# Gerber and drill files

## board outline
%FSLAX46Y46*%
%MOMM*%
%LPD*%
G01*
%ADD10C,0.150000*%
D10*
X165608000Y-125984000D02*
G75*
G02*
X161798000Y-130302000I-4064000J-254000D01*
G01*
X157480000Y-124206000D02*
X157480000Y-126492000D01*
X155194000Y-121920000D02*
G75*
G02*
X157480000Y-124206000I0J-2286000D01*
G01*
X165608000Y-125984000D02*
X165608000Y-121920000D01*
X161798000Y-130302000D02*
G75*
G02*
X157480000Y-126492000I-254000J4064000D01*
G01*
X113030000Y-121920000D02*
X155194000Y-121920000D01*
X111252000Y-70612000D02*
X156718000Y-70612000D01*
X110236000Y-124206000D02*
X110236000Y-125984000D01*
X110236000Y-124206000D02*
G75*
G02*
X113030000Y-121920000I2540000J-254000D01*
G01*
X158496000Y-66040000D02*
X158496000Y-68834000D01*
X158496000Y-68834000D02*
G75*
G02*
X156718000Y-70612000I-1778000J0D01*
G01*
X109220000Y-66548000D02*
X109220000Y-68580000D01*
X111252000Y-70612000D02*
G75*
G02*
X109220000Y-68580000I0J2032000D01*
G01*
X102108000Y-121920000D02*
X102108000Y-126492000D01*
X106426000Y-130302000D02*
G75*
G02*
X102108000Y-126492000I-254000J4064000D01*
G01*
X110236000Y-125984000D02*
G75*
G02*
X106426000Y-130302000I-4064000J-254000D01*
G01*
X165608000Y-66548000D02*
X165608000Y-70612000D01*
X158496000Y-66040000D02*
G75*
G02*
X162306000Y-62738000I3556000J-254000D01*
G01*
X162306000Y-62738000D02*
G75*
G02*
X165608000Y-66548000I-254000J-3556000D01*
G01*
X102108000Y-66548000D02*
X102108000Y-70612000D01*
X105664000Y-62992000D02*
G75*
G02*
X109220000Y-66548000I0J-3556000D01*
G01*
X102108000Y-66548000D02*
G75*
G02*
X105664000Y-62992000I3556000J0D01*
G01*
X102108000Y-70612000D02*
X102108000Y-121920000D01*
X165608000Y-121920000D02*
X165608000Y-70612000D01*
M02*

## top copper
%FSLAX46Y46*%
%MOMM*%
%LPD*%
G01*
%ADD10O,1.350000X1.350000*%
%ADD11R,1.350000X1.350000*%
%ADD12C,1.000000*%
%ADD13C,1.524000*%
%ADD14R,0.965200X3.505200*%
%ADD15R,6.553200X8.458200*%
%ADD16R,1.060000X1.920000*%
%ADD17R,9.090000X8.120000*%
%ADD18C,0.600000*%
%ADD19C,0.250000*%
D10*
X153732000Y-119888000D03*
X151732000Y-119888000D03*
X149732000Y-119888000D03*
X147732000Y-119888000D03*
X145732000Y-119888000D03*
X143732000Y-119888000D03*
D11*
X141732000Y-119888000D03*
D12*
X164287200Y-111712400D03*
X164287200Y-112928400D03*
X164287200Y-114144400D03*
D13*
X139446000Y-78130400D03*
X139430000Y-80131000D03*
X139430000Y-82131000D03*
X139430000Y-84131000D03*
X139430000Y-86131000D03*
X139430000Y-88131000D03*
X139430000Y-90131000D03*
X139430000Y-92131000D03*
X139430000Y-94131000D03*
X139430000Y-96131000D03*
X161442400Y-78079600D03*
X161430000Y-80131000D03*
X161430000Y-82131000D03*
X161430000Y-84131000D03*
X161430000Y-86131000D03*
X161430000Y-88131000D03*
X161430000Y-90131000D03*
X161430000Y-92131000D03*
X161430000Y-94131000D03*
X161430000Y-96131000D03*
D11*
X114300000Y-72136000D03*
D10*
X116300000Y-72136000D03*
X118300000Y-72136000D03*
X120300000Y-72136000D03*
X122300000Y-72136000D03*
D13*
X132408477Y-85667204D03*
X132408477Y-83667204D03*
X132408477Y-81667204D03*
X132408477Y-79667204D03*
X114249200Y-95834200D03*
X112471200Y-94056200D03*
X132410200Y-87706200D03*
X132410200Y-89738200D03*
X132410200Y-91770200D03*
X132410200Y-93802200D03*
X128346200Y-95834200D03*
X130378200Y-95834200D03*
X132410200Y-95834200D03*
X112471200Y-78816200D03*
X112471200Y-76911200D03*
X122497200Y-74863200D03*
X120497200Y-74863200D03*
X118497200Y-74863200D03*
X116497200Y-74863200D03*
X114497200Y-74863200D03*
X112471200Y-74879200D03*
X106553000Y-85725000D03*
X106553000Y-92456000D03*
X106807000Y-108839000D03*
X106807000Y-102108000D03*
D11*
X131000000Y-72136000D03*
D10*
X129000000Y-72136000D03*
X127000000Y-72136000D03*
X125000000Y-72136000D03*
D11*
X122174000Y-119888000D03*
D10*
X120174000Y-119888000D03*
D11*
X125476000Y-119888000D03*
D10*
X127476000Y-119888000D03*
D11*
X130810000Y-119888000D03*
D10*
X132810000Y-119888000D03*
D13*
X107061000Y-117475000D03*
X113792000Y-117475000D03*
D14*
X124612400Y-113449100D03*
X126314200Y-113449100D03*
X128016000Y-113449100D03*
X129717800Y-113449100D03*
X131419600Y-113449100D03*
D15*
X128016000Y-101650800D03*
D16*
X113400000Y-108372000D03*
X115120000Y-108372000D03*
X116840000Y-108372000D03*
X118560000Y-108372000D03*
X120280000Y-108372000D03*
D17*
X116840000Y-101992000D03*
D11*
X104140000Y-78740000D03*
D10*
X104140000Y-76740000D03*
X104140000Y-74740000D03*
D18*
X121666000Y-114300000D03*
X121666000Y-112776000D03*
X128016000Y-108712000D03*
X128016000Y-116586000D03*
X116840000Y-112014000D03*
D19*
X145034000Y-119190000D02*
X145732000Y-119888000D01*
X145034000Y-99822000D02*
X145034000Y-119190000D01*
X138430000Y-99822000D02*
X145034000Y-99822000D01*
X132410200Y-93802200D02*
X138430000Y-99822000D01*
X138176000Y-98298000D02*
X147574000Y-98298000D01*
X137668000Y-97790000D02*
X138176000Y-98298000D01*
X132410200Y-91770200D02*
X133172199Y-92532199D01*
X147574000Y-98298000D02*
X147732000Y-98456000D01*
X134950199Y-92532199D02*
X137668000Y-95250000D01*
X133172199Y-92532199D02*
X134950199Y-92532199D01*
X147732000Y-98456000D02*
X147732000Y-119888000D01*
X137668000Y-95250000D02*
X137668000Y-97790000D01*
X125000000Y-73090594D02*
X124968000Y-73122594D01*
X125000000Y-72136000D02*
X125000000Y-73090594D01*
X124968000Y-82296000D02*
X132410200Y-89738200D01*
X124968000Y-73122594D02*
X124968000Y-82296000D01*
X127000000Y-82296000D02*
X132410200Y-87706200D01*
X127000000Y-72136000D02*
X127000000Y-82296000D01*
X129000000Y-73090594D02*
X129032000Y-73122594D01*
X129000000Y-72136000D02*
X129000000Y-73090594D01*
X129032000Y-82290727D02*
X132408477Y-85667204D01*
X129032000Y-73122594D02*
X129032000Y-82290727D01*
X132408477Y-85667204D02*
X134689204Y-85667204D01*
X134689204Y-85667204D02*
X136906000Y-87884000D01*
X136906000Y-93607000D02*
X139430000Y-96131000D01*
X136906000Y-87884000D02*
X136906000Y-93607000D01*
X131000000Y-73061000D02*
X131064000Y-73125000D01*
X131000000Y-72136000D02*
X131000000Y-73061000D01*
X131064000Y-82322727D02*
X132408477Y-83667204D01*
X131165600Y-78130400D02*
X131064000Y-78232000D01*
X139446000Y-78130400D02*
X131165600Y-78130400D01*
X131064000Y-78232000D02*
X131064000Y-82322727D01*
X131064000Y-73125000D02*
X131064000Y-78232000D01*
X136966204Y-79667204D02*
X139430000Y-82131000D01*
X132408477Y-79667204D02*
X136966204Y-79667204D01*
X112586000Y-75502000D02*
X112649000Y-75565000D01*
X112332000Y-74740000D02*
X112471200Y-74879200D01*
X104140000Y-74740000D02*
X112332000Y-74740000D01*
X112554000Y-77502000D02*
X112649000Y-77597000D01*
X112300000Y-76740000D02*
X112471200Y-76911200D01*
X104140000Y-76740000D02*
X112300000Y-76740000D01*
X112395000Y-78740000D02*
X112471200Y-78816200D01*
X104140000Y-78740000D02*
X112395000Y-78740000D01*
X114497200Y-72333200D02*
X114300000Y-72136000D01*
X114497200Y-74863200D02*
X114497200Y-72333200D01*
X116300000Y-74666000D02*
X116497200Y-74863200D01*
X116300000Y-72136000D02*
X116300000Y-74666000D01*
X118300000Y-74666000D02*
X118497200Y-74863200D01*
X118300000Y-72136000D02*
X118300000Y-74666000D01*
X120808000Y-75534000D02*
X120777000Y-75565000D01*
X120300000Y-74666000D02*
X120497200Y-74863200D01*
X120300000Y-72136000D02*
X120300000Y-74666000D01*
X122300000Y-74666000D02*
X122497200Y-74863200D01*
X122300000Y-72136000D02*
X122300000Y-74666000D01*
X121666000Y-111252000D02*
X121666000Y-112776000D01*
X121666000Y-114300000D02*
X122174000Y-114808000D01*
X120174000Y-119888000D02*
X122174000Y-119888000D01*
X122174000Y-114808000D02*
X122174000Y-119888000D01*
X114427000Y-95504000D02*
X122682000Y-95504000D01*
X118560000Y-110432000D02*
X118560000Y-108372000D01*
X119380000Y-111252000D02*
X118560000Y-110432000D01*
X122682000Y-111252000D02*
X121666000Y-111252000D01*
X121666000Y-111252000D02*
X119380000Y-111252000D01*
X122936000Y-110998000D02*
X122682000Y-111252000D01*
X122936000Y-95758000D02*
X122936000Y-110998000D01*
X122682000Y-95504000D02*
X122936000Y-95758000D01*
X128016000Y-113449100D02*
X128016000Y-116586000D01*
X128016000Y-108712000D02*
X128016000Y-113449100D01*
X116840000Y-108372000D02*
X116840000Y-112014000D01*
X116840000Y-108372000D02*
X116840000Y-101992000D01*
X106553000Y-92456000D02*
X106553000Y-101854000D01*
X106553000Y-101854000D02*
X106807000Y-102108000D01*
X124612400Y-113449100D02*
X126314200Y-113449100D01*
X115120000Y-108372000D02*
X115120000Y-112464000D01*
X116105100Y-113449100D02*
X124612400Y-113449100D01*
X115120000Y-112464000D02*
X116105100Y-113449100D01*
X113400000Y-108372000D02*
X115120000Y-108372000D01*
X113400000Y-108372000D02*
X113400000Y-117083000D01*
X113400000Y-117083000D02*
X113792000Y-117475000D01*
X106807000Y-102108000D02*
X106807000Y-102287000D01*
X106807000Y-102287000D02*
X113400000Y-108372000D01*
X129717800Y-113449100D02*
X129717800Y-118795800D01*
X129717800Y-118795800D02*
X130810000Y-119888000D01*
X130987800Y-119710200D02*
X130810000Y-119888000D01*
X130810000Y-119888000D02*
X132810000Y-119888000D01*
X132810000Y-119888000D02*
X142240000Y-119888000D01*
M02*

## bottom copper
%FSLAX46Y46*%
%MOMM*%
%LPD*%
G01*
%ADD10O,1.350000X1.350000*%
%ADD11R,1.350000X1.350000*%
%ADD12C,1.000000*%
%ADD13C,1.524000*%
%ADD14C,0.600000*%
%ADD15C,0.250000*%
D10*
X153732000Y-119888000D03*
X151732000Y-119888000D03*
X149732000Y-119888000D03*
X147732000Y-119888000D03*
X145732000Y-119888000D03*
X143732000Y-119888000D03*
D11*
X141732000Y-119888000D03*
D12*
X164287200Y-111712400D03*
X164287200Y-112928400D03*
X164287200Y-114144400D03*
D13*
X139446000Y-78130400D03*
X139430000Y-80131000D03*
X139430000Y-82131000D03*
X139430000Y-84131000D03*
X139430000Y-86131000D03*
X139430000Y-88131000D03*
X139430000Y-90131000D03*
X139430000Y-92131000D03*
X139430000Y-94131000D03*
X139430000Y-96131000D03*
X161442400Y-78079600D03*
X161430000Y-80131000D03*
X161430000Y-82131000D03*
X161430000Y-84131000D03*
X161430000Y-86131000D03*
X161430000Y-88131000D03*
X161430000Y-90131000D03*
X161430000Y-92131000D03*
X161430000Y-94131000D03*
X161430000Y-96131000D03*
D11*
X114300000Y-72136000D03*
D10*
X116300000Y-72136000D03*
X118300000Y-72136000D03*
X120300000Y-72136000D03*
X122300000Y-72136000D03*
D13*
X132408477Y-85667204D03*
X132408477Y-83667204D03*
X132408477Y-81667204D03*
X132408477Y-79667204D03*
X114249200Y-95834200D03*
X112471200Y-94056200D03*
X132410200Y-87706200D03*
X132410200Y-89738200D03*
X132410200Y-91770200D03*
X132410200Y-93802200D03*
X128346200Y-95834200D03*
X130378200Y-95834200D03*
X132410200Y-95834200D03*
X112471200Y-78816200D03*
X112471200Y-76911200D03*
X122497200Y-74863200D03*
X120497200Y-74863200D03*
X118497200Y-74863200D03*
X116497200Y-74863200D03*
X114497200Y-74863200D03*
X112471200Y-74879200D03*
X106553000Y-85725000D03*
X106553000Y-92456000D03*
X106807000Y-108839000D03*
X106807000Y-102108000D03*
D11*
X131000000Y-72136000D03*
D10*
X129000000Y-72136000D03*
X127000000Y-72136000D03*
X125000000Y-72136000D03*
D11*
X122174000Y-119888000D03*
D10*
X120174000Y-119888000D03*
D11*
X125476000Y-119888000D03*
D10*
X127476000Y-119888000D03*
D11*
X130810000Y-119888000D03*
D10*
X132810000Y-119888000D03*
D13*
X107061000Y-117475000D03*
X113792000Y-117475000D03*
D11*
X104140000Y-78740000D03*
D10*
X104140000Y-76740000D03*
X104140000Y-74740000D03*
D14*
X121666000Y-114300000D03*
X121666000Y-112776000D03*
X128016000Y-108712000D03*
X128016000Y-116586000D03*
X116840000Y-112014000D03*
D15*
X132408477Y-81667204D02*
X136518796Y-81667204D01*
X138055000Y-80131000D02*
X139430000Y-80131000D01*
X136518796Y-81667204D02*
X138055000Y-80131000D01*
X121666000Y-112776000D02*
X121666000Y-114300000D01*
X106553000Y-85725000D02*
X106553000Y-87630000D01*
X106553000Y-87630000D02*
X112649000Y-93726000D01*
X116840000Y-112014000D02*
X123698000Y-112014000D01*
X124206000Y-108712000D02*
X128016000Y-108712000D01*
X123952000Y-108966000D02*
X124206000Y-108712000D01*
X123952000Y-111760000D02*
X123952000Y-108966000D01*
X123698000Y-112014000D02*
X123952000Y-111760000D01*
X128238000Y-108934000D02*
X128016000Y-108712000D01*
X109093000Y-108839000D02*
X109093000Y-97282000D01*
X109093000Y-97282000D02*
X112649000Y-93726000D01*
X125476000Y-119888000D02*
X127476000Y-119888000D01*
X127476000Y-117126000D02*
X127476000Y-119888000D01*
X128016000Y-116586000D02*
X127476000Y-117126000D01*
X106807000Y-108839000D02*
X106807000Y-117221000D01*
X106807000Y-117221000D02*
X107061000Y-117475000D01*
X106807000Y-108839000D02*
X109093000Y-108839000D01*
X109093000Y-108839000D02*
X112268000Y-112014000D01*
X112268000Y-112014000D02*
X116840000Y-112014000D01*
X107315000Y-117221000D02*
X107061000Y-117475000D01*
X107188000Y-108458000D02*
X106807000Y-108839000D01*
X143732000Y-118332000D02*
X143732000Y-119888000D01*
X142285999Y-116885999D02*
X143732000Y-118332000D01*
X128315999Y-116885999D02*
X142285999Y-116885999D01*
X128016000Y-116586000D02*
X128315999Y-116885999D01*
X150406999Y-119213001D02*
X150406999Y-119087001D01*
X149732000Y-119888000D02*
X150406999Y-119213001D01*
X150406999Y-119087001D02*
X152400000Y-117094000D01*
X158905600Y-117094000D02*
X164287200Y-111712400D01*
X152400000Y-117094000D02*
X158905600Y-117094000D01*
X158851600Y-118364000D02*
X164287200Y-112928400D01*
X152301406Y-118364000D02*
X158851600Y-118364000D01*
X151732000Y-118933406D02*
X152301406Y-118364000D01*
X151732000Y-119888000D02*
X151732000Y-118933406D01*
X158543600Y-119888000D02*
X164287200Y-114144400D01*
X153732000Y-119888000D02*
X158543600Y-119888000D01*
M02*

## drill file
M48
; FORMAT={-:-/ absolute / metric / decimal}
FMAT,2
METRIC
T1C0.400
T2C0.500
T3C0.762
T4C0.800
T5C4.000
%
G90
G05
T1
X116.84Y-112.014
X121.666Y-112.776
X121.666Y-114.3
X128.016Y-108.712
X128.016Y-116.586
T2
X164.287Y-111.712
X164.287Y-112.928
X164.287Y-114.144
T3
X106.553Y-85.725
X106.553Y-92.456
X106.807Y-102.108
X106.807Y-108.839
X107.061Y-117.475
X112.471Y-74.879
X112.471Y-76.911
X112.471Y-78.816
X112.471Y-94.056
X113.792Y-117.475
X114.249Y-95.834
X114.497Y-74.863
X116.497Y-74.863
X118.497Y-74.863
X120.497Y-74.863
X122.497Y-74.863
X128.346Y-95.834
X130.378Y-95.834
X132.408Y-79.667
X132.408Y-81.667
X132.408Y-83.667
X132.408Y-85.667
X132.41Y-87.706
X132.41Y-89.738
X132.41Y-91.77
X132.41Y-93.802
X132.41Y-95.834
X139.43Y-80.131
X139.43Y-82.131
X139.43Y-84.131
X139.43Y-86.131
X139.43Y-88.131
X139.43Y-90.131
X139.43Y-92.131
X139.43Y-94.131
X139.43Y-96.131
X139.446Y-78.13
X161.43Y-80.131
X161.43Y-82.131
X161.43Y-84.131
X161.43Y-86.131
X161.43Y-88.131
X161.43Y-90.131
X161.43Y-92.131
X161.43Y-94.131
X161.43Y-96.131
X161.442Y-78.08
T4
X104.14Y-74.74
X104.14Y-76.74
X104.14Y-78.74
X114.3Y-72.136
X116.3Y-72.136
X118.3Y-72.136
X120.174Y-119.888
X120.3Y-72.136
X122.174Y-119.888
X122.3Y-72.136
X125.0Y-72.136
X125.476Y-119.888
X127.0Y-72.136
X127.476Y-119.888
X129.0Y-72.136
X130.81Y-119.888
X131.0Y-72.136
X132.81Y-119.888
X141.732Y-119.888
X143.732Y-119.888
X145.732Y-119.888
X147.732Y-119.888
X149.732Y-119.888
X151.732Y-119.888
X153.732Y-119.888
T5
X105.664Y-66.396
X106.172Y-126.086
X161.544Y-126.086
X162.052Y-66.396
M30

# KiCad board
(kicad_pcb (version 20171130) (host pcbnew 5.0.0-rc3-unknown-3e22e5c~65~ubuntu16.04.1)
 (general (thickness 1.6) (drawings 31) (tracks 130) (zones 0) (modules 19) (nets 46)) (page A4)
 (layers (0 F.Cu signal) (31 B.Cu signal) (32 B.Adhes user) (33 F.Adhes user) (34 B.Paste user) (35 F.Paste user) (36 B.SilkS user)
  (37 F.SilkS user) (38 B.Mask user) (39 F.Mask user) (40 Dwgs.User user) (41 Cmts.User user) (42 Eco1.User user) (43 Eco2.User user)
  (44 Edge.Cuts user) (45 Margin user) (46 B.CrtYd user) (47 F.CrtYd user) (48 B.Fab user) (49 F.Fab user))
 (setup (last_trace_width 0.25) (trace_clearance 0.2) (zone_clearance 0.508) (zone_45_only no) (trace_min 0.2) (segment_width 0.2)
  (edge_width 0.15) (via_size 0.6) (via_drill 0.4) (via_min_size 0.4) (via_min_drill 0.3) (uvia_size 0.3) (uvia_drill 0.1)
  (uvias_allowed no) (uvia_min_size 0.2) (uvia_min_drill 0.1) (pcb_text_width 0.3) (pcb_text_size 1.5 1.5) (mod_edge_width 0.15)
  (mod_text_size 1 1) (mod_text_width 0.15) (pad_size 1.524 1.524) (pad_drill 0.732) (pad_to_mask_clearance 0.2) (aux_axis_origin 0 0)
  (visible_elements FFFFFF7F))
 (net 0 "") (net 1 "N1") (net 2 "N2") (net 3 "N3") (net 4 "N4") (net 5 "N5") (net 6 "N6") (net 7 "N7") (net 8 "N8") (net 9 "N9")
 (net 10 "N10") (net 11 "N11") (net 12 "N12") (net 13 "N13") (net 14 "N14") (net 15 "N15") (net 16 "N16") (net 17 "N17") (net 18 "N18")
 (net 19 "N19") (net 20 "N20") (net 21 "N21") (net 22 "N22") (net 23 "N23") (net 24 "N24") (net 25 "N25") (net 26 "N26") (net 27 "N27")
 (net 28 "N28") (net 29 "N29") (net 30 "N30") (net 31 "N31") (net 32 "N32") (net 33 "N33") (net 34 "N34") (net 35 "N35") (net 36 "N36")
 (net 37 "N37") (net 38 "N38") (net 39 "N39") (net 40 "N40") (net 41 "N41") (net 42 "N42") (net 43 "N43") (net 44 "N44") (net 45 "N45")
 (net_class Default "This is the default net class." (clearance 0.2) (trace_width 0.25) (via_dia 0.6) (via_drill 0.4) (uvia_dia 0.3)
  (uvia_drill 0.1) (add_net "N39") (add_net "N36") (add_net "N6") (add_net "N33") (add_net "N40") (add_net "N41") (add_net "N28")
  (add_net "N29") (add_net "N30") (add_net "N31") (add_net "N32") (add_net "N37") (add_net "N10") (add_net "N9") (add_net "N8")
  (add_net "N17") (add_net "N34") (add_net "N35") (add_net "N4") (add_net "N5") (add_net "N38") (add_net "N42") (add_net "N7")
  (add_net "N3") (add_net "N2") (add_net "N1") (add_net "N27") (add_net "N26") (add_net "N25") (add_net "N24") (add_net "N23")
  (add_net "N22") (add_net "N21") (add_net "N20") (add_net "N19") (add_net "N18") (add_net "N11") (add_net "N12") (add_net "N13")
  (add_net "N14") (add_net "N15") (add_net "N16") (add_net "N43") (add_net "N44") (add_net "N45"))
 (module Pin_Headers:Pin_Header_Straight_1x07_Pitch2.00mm (layer F.Cu) (at 141.732 119.888 90)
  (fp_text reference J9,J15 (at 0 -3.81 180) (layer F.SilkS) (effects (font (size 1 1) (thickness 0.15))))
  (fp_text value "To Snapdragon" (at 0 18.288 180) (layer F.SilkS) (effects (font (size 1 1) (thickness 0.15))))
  (pad 5 thru_hole oval (at 0 12 90) (size 1.35 1.35) (drill 0.8) (layers *.Cu *.Mask) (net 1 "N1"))
  (pad 4 thru_hole oval (at 0 10 90) (size 1.35 1.35) (drill 0.8) (layers *.Cu *.Mask) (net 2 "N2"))
  (pad 3 thru_hole oval (at 0 8 90) (size 1.35 1.35) (drill 0.8) (layers *.Cu *.Mask) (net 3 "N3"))
  (pad 6 thru_hole oval (at 0 6 90) (size 1.35 1.35) (drill 0.8) (layers *.Cu *.Mask) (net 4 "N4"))
  (pad 7 thru_hole oval (at 0 4 90) (size 1.35 1.35) (drill 0.8) (layers *.Cu *.Mask) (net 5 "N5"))
  (pad 2 thru_hole oval (at 0 2 90) (size 1.35 1.35) (drill 0.8) (layers *.Cu *.Mask) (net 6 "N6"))
  (pad 1 thru_hole rect (at 0 0 90) (size 1.35 1.35) (drill 0.8) (layers *.Cu *.Mask) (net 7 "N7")))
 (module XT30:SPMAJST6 (layer F.Cu) (at 163.576 113.792 270)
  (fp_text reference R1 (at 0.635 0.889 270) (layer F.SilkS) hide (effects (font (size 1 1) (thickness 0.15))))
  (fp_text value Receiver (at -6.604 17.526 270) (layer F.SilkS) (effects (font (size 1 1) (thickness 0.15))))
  (pad 1 thru_hole circle (at -2.0796 -0.7112 270) (size 1 1) (drill 0.5) (layers *.Cu *.Mask) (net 3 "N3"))
  (pad 2 thru_hole circle (at -0.8636 -0.7112 270) (size 1 1) (drill 0.5) (layers *.Cu *.Mask) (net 2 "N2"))
  (pad 3 thru_hole circle (at 0.3524 -0.7112 270) (size 1 1) (drill 0.5) (layers *.Cu *.Mask) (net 1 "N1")))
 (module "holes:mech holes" (layer F.Cu) (at 162.052 129.286)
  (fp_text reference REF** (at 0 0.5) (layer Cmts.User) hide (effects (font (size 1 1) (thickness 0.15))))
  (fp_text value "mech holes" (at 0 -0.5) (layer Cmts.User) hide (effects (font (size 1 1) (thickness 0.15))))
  (pad "" np_thru_hole circle (at -0.508 -3.2004) (size 4 4) (drill 4) (layers *.Cu *.Mask)))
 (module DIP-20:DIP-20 (layer F.Cu) (at 138.176 104.14)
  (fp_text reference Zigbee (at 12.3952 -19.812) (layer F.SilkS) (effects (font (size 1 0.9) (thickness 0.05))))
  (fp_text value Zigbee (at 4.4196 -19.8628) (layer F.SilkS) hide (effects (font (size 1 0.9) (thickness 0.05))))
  (pad 1 thru_hole circle (at 1.27 -26.0096) (size 1.524 1.524) (drill 0.762) (layers *.Cu *.Mask F.SilkS) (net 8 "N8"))
  (pad 2 thru_hole circle (at 1.254 -24.009) (size 1.524 1.524) (drill 0.762) (layers *.Cu *.Mask F.SilkS) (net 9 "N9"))
  (pad 3 thru_hole circle (at 1.254 -22.009) (size 1.524 1.524) (drill 0.762) (layers *.Cu *.Mask F.SilkS) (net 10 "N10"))
  (pad 4 thru_hole circle (at 1.254 -20.009) (size 1.524 1.524) (drill 0.762) (layers *.Cu *.Mask F.SilkS) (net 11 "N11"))
  (pad 5 thru_hole circle (at 1.254 -18.009) (size 1.524 1.524) (drill 0.762) (layers *.Cu *.Mask F.SilkS) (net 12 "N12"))
  (pad 6 thru_hole circle (at 1.254 -16.009) (size 1.524 1.524) (drill 0.762) (layers *.Cu *.Mask F.SilkS) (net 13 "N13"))
  (pad 7 thru_hole circle (at 1.254 -14.009) (size 1.524 1.524) (drill 0.762) (layers *.Cu *.Mask F.SilkS) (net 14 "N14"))
  (pad 8 thru_hole circle (at 1.254 -12.009) (size 1.524 1.524) (drill 0.762) (layers *.Cu *.Mask F.SilkS) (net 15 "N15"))
  (pad 9 thru_hole circle (at 1.254 -10.009) (size 1.524 1.524) (drill 0.762) (layers *.Cu *.Mask F.SilkS) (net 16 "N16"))
  (pad 10 thru_hole circle (at 1.254 -8.009) (size 1.524 1.524) (drill 0.762) (layers *.Cu *.Mask F.SilkS) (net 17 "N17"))
  (pad 20 thru_hole circle (at 23.2664 -26.0604) (size 1.524 1.524) (drill 0.762) (layers *.Cu *.Mask F.SilkS) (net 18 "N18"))
  (pad 19 thru_hole circle (at 23.254 -24.009) (size 1.524 1.524) (drill 0.762) (layers *.Cu *.Mask F.SilkS) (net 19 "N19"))
  (pad 18 thru_hole circle (at 23.254 -22.009) (size 1.524 1.524) (drill 0.762) (layers *.Cu *.Mask F.SilkS) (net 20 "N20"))
  (pad 17 thru_hole circle (at 23.254 -20.009) (size 1.524 1.524) (drill 0.762) (layers *.Cu *.Mask F.SilkS) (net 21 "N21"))
  (pad 16 thru_hole circle (at 23.254 -18.009) (size 1.524 1.524) (drill 0.762) (layers *.Cu *.Mask F.SilkS) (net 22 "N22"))
  (pad 15 thru_hole circle (at 23.254 -16.009) (size 1.524 1.524) (drill 0.762) (layers *.Cu *.Mask F.SilkS) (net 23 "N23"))
  (pad 14 thru_hole circle (at 23.254 -14.009) (size 1.524 1.524) (drill 0.762) (layers *.Cu *.Mask F.SilkS) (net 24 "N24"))
  (pad 13 thru_hole circle (at 23.254 -12.009) (size 1.524 1.524) (drill 0.762) (layers *.Cu *.Mask F.SilkS) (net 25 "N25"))
  (pad 12 thru_hole circle (at 23.254 -10.009) (size 1.524 1.524) (drill 0.762) (layers *.Cu *.Mask F.SilkS) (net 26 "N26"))
  (pad 11 thru_hole circle (at 23.254 -8.009) (size 1.524 1.524) (drill 0.762) (layers *.Cu *.Mask F.SilkS) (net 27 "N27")))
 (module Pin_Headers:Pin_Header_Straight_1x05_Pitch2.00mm (layer F.Cu) (at 114.3 72.136 90)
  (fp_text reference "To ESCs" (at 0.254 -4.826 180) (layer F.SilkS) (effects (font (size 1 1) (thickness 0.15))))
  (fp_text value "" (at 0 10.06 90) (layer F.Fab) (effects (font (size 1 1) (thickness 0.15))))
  (pad 1 thru_hole rect (at 0 0 90) (size 1.35 1.35) (drill 0.8) (layers *.Cu *.Mask) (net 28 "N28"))
  (pad 2 thru_hole oval (at 0 2 90) (size 1.35 1.35) (drill 0.8) (layers *.Cu *.Mask) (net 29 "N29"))
  (pad 3 thru_hole oval (at 0 4 90) (size 1.35 1.35) (drill 0.8) (layers *.Cu *.Mask) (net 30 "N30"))
  (pad 4 thru_hole oval (at 0 6 90) (size 1.35 1.35) (drill 0.8) (layers *.Cu *.Mask) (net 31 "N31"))
  (pad 5 thru_hole oval (at 0 8 90) (size 1.35 1.35) (drill 0.8) (layers *.Cu *.Mask) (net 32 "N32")))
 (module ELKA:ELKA (layer F.Cu) (at 121.666 85.852)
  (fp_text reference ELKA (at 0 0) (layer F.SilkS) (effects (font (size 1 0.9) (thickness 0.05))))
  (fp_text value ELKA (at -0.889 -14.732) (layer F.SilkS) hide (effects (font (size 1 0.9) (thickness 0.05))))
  (pad D thru_hole circle (at 10.742477 -0.184796) (size 1.524 1.524) (drill 0.762) (layers *.Cu *.Mask B.SilkS) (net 17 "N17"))
  (pad C thru_hole circle (at 10.742477 -2.184796) (size 1.524 1.524) (drill 0.762) (layers *.Cu *.Mask B.SilkS) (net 8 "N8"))
  (pad B thru_hole circle (at 10.742477 -4.184796) (size 1.524 1.524) (drill 0.762) (layers *.Cu *.Mask B.SilkS) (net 9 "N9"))
  (pad A thru_hole circle (at 10.742477 -6.184796) (size 1.524 1.524) (drill 0.762) (layers *.Cu *.Mask B.SilkS) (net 10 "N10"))
  (pad 12 thru_hole circle (at -7.4168 9.9822) (size 1.524 1.524) (drill 0.762) (layers *.Cu *.Mask B.SilkS) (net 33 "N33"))
  (pad 11 thru_hole circle (at -9.1948 8.2042 270) (size 1.524 1.524) (drill 0.762) (layers *.Cu *.Mask B.SilkS) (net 6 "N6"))
  (pad E thru_hole circle (at 10.7442 1.8542 270) (size 1.524 1.524) (drill 0.762) (layers *.Cu *.Mask B.SilkS) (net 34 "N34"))
  (pad F thru_hole circle (at 10.7442 3.8862 270) (size 1.524 1.524) (drill 0.762) (layers *.Cu *.Mask B.SilkS) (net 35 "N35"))
  (pad G thru_hole circle (at 10.7442 5.9182 270) (size 1.524 1.524) (drill 0.762) (layers *.Cu *.Mask B.SilkS) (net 4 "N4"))
  (pad H thru_hole circle (at 10.7442 7.9502 270) (size 1.524 1.524) (drill 0.762) (layers *.Cu *.Mask B.SilkS) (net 5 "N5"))
  (pad 10 thru_hole circle (at 6.6802 9.9822 270) (size 1.524 1.524) (drill 0.762) (layers *.Cu *.Mask B.SilkS) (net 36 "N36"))
  (pad 9 thru_hole circle (at 8.7122 9.9822 270) (size 1.524 1.524) (drill 0.762) (layers *.Cu *.Mask B.SilkS) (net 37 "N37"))
  (pad I thru_hole circle (at 10.7442 9.9822 270) (size 1.524 1.524) (drill 0.762) (layers *.Cu *.Mask B.SilkS) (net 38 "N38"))
  (pad 1 thru_hole circle (at -9.1948 -7.0358 270) (size 1.524 1.524) (drill 0.762) (layers *.Cu *.Mask B.SilkS) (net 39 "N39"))
  (pad 2 thru_hole circle (at -9.1948 -8.9408 270) (size 1.524 1.524) (drill 0.762) (layers *.Cu *.Mask B.SilkS) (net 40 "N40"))
  (pad 8 thru_hole circle (at 0.8312 -10.9888 270) (size 1.524 1.524) (drill 0.762) (layers *.Cu *.Mask B.SilkS) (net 32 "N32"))
  (pad 7 thru_hole circle (at -1.1688 -10.9888 270) (size 1.524 1.524) (drill 0.762) (layers *.Cu *.Mask B.SilkS) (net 31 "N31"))
  (pad 6 thru_hole circle (at -3.1688 -10.9888 270) (size 1.524 1.524) (drill 0.762) (layers *.Cu *.Mask B.SilkS) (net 30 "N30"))
  (pad 5 thru_hole circle (at -5.1688 -10.9888 270) (size 1.524 1.524) (drill 0.762) (layers *.Cu *.Mask B.SilkS) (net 29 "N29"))
  (pad 4 thru_hole circle (at -7.1688 -10.9888 270) (size 1.524 1.524) (drill 0.762) (layers *.Cu *.Mask B.SilkS) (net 28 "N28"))
  (pad 3 thru_hole circle (at -9.1948 -10.9728 270) (size 1.524 1.524) (drill 0.762) (layers *.Cu *.Mask B.SilkS) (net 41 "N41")))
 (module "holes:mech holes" (layer F.Cu) (at 106.172 69.596)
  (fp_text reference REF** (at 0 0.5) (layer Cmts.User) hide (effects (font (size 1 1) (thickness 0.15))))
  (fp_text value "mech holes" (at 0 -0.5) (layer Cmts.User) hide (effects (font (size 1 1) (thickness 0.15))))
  (pad "" np_thru_hole circle (at -0.508 -3.2004) (size 4 4) (drill 4) (layers *.Cu *.Mask)))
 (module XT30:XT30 (layer F.Cu) (at 112.522 87.122 270)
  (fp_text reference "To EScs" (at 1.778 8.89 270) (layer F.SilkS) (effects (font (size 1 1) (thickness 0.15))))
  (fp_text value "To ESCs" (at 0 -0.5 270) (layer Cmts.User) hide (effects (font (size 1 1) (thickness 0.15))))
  (pad 1 thru_hole circle (at -1.397 5.969 270) (size 1.524 1.524) (drill 0.762) (layers *.Cu *.Mask) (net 6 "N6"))
  (pad 2 thru_hole circle (at 5.334 5.969 270) (size 1.524 1.524) (drill 0.762) (layers *.Cu *.Mask) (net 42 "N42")))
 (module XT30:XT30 (layer F.Cu) (at 100.838 107.442 90)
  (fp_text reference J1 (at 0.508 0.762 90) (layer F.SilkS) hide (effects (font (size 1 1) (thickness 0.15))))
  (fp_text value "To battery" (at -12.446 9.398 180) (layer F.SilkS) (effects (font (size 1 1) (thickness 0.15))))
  (pad 1 thru_hole circle (at -1.397 5.969 90) (size 1.524 1.524) (drill 0.762) (layers *.Cu *.Mask) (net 6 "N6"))
  (pad 2 thru_hole circle (at 5.334 5.969 90) (size 1.524 1.524) (drill 0.762) (layers *.Cu *.Mask) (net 42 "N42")))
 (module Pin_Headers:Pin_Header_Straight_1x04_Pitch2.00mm (layer F.Cu) (at 131 72.136 270)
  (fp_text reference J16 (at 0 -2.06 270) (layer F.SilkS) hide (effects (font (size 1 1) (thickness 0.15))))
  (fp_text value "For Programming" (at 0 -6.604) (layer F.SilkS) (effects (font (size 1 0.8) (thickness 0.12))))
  (pad 1 thru_hole rect (at 0 0 270) (size 1.35 1.35) (drill 0.8) (layers *.Cu *.Mask) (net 8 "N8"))
  (pad 2 thru_hole oval (at 0 2 270) (size 1.35 1.35) (drill 0.8) (layers *.Cu *.Mask) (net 17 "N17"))
  (pad 3 thru_hole oval (at 0 4 270) (size 1.35 1.35) (drill 0.8) (layers *.Cu *.Mask) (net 34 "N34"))
  (pad 4 thru_hole oval (at 0 6 270) (size 1.35 1.35) (drill 0.8) (layers *.Cu *.Mask) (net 35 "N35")))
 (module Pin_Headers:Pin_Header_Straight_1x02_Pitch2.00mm (layer F.Cu) (at 122.174 119.888 270)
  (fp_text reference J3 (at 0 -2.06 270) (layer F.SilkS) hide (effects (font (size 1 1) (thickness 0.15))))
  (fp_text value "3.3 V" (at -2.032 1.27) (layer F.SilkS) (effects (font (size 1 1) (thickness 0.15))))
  (pad 1 thru_hole rect (at 0 0 270) (size 1.35 1.35) (drill 0.8) (layers *.Cu *.Mask) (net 33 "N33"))
  (pad 2 thru_hole oval (at 0 2 270) (size 1.35 1.35) (drill 0.8) (layers *.Cu *.Mask) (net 33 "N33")))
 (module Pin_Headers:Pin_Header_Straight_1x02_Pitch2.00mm (layer F.Cu) (at 125.476 119.888 90)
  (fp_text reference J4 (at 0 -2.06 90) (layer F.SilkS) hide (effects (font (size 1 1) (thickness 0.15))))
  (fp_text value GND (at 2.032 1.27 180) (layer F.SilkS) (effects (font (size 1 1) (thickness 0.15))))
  (pad 1 thru_hole rect (at 0 0 90) (size 1.35 1.35) (drill 0.8) (layers *.Cu *.Mask) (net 6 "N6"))
  (pad 2 thru_hole oval (at 0 2 90) (size 1.35 1.35) (drill 0.8) (layers *.Cu *.Mask) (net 6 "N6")))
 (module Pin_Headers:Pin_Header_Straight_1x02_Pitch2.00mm (layer F.Cu) (at 130.81 119.888 90)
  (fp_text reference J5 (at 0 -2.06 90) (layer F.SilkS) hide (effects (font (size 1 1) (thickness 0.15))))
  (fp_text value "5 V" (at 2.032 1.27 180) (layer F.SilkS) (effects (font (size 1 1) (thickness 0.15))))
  (pad 1 thru_hole rect (at 0 0 90) (size 1.35 1.35) (drill 0.8) (layers *.Cu *.Mask) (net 7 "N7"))
  (pad 2 thru_hole oval (at 0 2 90) (size 1.35 1.35) (drill 0.8) (layers *.Cu *.Mask) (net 7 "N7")))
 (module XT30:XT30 (layer F.Cu) (at 108.458 111.506)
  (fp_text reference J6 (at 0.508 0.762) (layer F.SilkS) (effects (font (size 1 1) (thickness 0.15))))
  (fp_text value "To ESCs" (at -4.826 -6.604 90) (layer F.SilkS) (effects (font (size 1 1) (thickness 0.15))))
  (pad 1 thru_hole circle (at -1.397 5.969) (size 1.524 1.524) (drill 0.762) (layers *.Cu *.Mask) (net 6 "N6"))
  (pad 2 thru_hole circle (at 5.334 5.969) (size 1.524 1.524) (drill 0.762) (layers *.Cu *.Mask) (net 42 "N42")))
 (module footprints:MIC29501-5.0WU (layer F.Cu) (at 128.016 104.394)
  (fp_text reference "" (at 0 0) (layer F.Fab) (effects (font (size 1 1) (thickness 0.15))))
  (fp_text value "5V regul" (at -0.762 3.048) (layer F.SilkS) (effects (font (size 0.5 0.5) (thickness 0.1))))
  (pad 1 smd rect (at -3.4036 9.0551) (size 0.9652 3.5052) (layers F.Cu F.Paste F.Mask) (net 42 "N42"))
  (pad 2 smd rect (at -1.7018 9.0551) (size 0.9652 3.5052) (layers F.Cu F.Paste F.Mask) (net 42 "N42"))
  (pad 3 smd rect (at 0 9.0551) (size 0.9652 3.5052) (layers F.Cu F.Paste F.Mask) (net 6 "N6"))
  (pad 4 smd rect (at 1.7018 9.0551) (size 0.9652 3.5052) (layers F.Cu F.Paste F.Mask) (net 7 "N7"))
  (pad 5 smd rect (at 3.4036 9.0551) (size 0.9652 3.5052) (layers F.Cu F.Paste F.Mask) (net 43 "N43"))
  (pad 6 smd rect (at 0 -2.7432) (size 6.5532 8.4582) (layers F.Cu F.Paste F.Mask) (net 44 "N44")))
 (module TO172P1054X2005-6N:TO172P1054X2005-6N (layer F.Cu) (at 116.84 103.632)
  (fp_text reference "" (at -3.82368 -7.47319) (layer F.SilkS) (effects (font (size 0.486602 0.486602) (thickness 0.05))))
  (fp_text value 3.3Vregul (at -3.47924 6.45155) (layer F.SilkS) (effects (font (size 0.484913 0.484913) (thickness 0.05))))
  (pad 1 smd rect (at -3.44 4.74 90) (size 1.92 1.06) (layers F.Cu F.Paste F.Mask) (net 42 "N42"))
  (pad 2 smd rect (at -1.72 4.74 90) (size 1.92 1.06) (layers F.Cu F.Paste F.Mask) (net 42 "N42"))
  (pad 3 smd rect (at 0 4.74 90) (size 1.92 1.06) (layers F.Cu F.Paste F.Mask) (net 6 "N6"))
  (pad 4 smd rect (at 1.72 4.74 90) (size 1.92 1.06) (layers F.Cu F.Paste F.Mask) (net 33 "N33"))
  (pad 5 smd rect (at 3.44 4.74 90) (size 1.92 1.06) (layers F.Cu F.Paste F.Mask) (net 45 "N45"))
  (pad 6 smd rect (at 0 -1.64 90) (size 8.12 9.09) (layers F.Cu F.Paste F.Mask) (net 6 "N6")))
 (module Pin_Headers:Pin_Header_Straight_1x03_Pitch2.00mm (layer F.Cu) (at 104.14 78.74 180)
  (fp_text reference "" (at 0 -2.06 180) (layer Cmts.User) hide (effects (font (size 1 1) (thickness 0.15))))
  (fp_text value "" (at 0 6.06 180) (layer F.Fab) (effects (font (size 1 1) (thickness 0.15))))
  (pad 1 thru_hole rect (at 0 0 180) (size 1.35 1.35) (drill 0.8) (layers *.Cu *.Mask) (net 39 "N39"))
  (pad 2 thru_hole oval (at 0 2 180) (size 1.35 1.35) (drill 0.8) (layers *.Cu *.Mask) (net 40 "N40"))
  (pad 3 thru_hole oval (at 0 4 180) (size 1.35 1.35) (drill 0.8) (layers *.Cu *.Mask) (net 41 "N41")))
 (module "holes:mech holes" (layer F.Cu) (at 162.56 69.596)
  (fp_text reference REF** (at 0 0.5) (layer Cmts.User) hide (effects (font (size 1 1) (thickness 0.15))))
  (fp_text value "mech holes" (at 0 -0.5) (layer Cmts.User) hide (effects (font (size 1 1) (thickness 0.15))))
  (pad "" np_thru_hole circle (at -0.508 -3.2004) (size 4 4) (drill 4) (layers *.Cu *.Mask)))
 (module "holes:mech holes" (layer F.Cu) (at 106.68 129.286)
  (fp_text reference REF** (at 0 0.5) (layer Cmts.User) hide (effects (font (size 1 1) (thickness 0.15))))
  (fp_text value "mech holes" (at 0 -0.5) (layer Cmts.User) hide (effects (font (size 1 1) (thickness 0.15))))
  (pad "" np_thru_hole circle (at -0.508 -3.2004) (size 4 4) (drill 4) (layers *.Cu *.Mask)))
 (gr_arc (start 161.544 126.238) (end 165.608 125.984) (angle 90) (layer Edge.Cuts) (width 0.15))
 (gr_line (start 157.48 124.206) (end 157.48 126.492) (angle 90) (layer Edge.Cuts) (width 0.15))
 (gr_arc (start 155.194 124.206) (end 155.194 121.92) (angle 90) (layer Edge.Cuts) (width 0.15))
 (gr_line (start 165.608 125.984) (end 165.608 121.92) (angle 90) (layer Edge.Cuts) (width 0.15))
 (gr_arc (start 161.544 126.238) (end 161.798 130.302) (angle 90) (layer Edge.Cuts) (width 0.15))
 (gr_line (start 113.03 121.92) (end 155.194 121.92) (angle 90) (layer Edge.Cuts) (width 0.15))
 (gr_line (start 111.252 70.612) (end 156.718 70.612) (angle 90) (layer Edge.Cuts) (width 0.15))
 (gr_line (start 110.236 124.206) (end 110.236 125.984) (angle 90) (layer Edge.Cuts) (width 0.15))
 (gr_arc (start 112.776 124.46) (end 110.236 124.206) (angle 90) (layer Edge.Cuts) (width 0.15))
 (gr_line (start 158.496 66.04) (end 158.496 68.834) (angle 90) (layer Edge.Cuts) (width 0.15))
 (gr_arc (start 156.718 68.834) (end 158.496 68.834) (angle 90) (layer Edge.Cuts) (width 0.15))
 (gr_line (start 109.22 66.548) (end 109.22 68.58) (angle 90) (layer Edge.Cuts) (width 0.15))
 (gr_arc (start 111.252 68.58) (end 111.252 70.612) (angle 90) (layer Edge.Cuts) (width 0.15))
 (gr_line (start 102.108 121.92) (end 102.108 126.492) (angle 90) (layer Edge.Cuts) (width 0.15))
 (gr_arc (start 106.172 126.238) (end 106.426 130.302) (angle 90) (layer Edge.Cuts) (width 0.15))
 (gr_arc (start 106.172 126.238) (end 110.236 125.984) (angle 90) (layer Edge.Cuts) (width 0.15))
 (gr_line (start 165.608 66.548) (end 165.608 70.612) (angle 90) (layer Edge.Cuts) (width 0.15))
 (gr_arc (start 162.052 66.294) (end 158.496 66.04) (angle 90) (layer Edge.Cuts) (width 0.15))
 (gr_arc (start 162.052 66.294) (end 162.306 62.738) (angle 90) (layer Edge.Cuts) (width 0.15))
 (gr_line (start 102.108 66.548) (end 102.108 70.612) (angle 90) (layer Edge.Cuts) (width 0.15))
 (gr_arc (start 105.664 66.548) (end 105.664 62.992) (angle 90) (layer Edge.Cuts) (width 0.15))
 (gr_arc (start 105.664 66.548) (end 102.108 66.548) (angle 90) (layer Edge.Cuts) (width 0.15))
 (gr_line (start 102.108 70.612) (end 102.108 121.92) (angle 90) (layer Edge.Cuts) (width 0.15))
 (gr_line (start 165.608 121.92) (end 165.608 70.612) (angle 90) (layer Edge.Cuts) (width 0.15))
 (segment (start 145.034 119.19) (end 145.732 119.888) (width 0.25) (layer F.Cu) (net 5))
 (segment (start 145.034 99.822) (end 145.034 119.19) (width 0.25) (layer F.Cu) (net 5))
 (segment (start 138.43 99.822) (end 145.034 99.822) (width 0.25) (layer F.Cu) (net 5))
 (segment (start 132.4102 93.8022) (end 138.43 99.822) (width 0.25) (layer F.Cu) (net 5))
 (segment (start 138.176 98.298) (end 147.574 98.298) (width 0.25) (layer F.Cu) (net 4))
 (segment (start 137.668 97.79) (end 138.176 98.298) (width 0.25) (layer F.Cu) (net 4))
 (segment (start 132.4102 91.7702) (end 133.172199 92.532199) (width 0.25) (layer F.Cu) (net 4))
 (segment (start 147.574 98.298) (end 147.732 98.456) (width 0.25) (layer F.Cu) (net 4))
 (segment (start 134.950199 92.532199) (end 137.668 95.25) (width 0.25) (layer F.Cu) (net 4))
 (segment (start 133.172199 92.532199) (end 134.950199 92.532199) (width 0.25) (layer F.Cu) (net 4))
 (segment (start 147.732 98.456) (end 147.732 119.888) (width 0.25) (layer F.Cu) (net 4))
 (segment (start 137.668 95.25) (end 137.668 97.79) (width 0.25) (layer F.Cu) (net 4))
 (segment (start 125 73.090594) (end 124.968 73.122594) (width 0.25) (layer F.Cu) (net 35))
 (segment (start 125 72.136) (end 125 73.090594) (width 0.25) (layer F.Cu) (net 35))
 (segment (start 124.968 82.296) (end 132.4102 89.7382) (width 0.25) (layer F.Cu) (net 35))
 (segment (start 124.968 73.122594) (end 124.968 82.296) (width 0.25) (layer F.Cu) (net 35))
 (segment (start 127 82.296) (end 132.4102 87.7062) (width 0.25) (layer F.Cu) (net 34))
 (segment (start 127 72.136) (end 127 82.296) (width 0.25) (layer F.Cu) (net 34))
 (segment (start 129 73.090594) (end 129.032 73.122594) (width 0.25) (layer F.Cu) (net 17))
 (segment (start 129 72.136) (end 129 73.090594) (width 0.25) (layer F.Cu) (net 17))
 (segment (start 129.032 82.290727) (end 132.408477 85.667204) (width 0.25) (layer F.Cu) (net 17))
 (segment (start 129.032 73.122594) (end 129.032 82.290727) (width 0.25) (layer F.Cu) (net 17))
 (segment (start 132.408477 85.667204) (end 134.689204 85.667204) (width 0.25) (layer F.Cu) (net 17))
 (segment (start 134.689204 85.667204) (end 136.906 87.884) (width 0.25) (layer F.Cu) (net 17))
 (segment (start 136.906 93.607) (end 139.43 96.131) (width 0.25) (layer F.Cu) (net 17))
 (segment (start 136.906 87.884) (end 136.906 93.607) (width 0.25) (layer F.Cu) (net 17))
 (segment (start 131 73.061) (end 131.064 73.125) (width 0.25) (layer F.Cu) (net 8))
 (segment (start 131 72.136) (end 131 73.061) (width 0.25) (layer F.Cu) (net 8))
 (segment (start 131.064 82.322727) (end 132.408477 83.667204) (width 0.25) (layer F.Cu) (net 8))
 (segment (start 131.1656 78.1304) (end 131.064 78.232) (width 0.25) (layer F.Cu) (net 8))
 (segment (start 139.446 78.1304) (end 131.1656 78.1304) (width 0.25) (layer F.Cu) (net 8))
 (segment (start 131.064 78.232) (end 131.064 82.322727) (width 0.25) (layer F.Cu) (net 8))
 (segment (start 131.064 73.125) (end 131.064 78.232) (width 0.25) (layer F.Cu) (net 8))
 (segment (start 132.408477 81.667204) (end 136.518796 81.667204) (width 0.25) (layer B.Cu) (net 9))
 (segment (start 138.055 80.131) (end 139.43 80.131) (width 0.25) (layer B.Cu) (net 9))
 (segment (start 136.518796 81.667204) (end 138.055 80.131) (width 0.25) (layer B.Cu) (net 9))
 (segment (start 136.966204 79.667204) (end 139.43 82.131) (width 0.25) (layer F.Cu) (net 10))
 (segment (start 132.408477 79.667204) (end 136.966204 79.667204) (width 0.25) (layer F.Cu) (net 10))
 (segment (start 112.586 75.502) (end 112.649 75.565) (width 0.25) (layer F.Cu) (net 41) (status 30))
 (segment (start 112.332 74.74) (end 112.4712 74.8792) (width 0.25) (layer F.Cu) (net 41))
 (segment (start 104.14 74.74) (end 112.332 74.74) (width 0.25) (layer F.Cu) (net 41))
 (segment (start 112.554 77.502) (end 112.649 77.597) (width 0.25) (layer F.Cu) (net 40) (status 30))
 (segment (start 112.3 76.74) (end 112.4712 76.9112) (width 0.25) (layer F.Cu) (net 40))
 (segment (start 104.14 76.74) (end 112.3 76.74) (width 0.25) (layer F.Cu) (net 40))
 (segment (start 112.395 78.74) (end 112.4712 78.8162) (width 0.25) (layer F.Cu) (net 39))
 (segment (start 104.14 78.74) (end 112.395 78.74) (width 0.25) (layer F.Cu) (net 39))
 (segment (start 114.4972 72.3332) (end 114.3 72.136) (width 0.25) (layer F.Cu) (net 28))
 (segment (start 114.4972 74.8632) (end 114.4972 72.3332) (width 0.25) (layer F.Cu) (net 28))
 (segment (start 116.3 74.666) (end 116.4972 74.8632) (width 0.25) (layer F.Cu) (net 29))
 (segment (start 116.3 72.136) (end 116.3 74.666) (width 0.25) (layer F.Cu) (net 29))
 (segment (start 118.3 74.666) (end 118.4972 74.8632) (width 0.25) (layer F.Cu) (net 30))
 (segment (start 118.3 72.136) (end 118.3 74.666) (width 0.25) (layer F.Cu) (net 30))
 (segment (start 120.808 75.534) (end 120.777 75.565) (width 0.25) (layer F.Cu) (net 31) (status 30))
 (segment (start 120.3 74.666) (end 120.4972 74.8632) (width 0.25) (layer F.Cu) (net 31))
 (segment (start 120.3 72.136) (end 120.3 74.666) (width 0.25) (layer F.Cu) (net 31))
 (segment (start 122.3 74.666) (end 122.4972 74.8632) (width 0.25) (layer F.Cu) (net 32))
 (segment (start 122.3 72.136) (end 122.3 74.666) (width 0.25) (layer F.Cu) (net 32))
 (segment (start 121.666 111.252) (end 121.666 112.776) (width 0.25) (layer F.Cu) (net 33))
 (segment (start 121.666 114.3) (end 122.174 114.808) (width 0.25) (layer F.Cu) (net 33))
 (via (at 121.666 114.3) (size 0.6) (drill 0.4) (layers F.Cu B.Cu) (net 33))
 (segment (start 121.666 112.776) (end 121.666 114.3) (width 0.25) (layer B.Cu) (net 33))
 (via (at 121.666 112.776) (size 0.6) (drill 0.4) (layers F.Cu B.Cu) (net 33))
 (segment (start 120.174 119.888) (end 122.174 119.888) (width 0.25) (layer F.Cu) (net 33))
 (segment (start 122.174 114.808) (end 122.174 119.888) (width 0.25) (layer F.Cu) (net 33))
 (segment (start 114.427 95.504) (end 122.682 95.504) (width 0.25) (layer F.Cu) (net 33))
 (segment (start 118.56 110.432) (end 118.56 108.372) (width 0.25) (layer F.Cu) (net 33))
 (segment (start 119.38 111.252) (end 118.56 110.432) (width 0.25) (layer F.Cu) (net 33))
 (segment (start 122.682 111.252) (end 121.666 111.252) (width 0.25) (layer F.Cu) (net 33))
 (segment (start 121.666 111.252) (end 119.38 111.252) (width 0.25) (layer F.Cu) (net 33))
 (segment (start 122.936 110.998) (end 122.682 111.252) (width 0.25) (layer F.Cu) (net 33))
 (segment (start 122.936 95.758) (end 122.936 110.998) (width 0.25) (layer F.Cu) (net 33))
 (segment (start 122.682 95.504) (end 122.936 95.758) (width 0.25) (layer F.Cu) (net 33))
 (segment (start 106.553 85.725) (end 106.553 87.63) (width 0.25) (layer B.Cu) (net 6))
 (segment (start 106.553 87.63) (end 112.649 93.726) (width 0.25) (layer B.Cu) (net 6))
 (segment (start 116.84 112.014) (end 123.698 112.014) (width 0.25) (layer B.Cu) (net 6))
 (segment (start 124.206 108.712) (end 128.016 108.712) (width 0.25) (layer B.Cu) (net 6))
 (segment (start 123.952 108.966) (end 124.206 108.712) (width 0.25) (layer B.Cu) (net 6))
 (segment (start 123.952 111.76) (end 123.952 108.966) (width 0.25) (layer B.Cu) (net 6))
 (segment (start 123.698 112.014) (end 123.952 111.76) (width 0.25) (layer B.Cu) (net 6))
 (segment (start 128.238 108.934) (end 128.016 108.712) (width 0.25) (layer B.Cu) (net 6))
 (via (at 128.016 108.712) (size 0.6) (drill 0.4) (layers F.Cu B.Cu) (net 6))
 (segment (start 109.093 108.839) (end 109.093 97.282) (width 0.25) (layer B.Cu) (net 6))
 (segment (start 109.093 97.282) (end 112.649 93.726) (width 0.25) (layer B.Cu) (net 6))
 (segment (start 125.476 119.888) (end 127.476 119.888) (width 0.25) (layer B.Cu) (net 6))
 (segment (start 128.016 113.4491) (end 128.016 116.586) (width 0.25) (layer F.Cu) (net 6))
 (segment (start 127.476 117.126) (end 127.476 119.888) (width 0.25) (layer B.Cu) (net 6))
 (segment (start 128.016 116.586) (end 127.476 117.126) (width 0.25) (layer B.Cu) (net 6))
 (via (at 128.016 116.586) (size 0.6) (drill 0.4) (layers F.Cu B.Cu) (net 6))
 (segment (start 106.807 108.839) (end 106.807 117.221) (width 0.25) (layer B.Cu) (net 6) (status 10))
 (segment (start 106.807 117.221) (end 107.061 117.475) (width 0.25) (layer B.Cu) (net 6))
 (segment (start 128.016 108.712) (end 128.016 113.4491) (width 0.25) (layer F.Cu) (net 6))
 (segment (start 116.84 108.372) (end 116.84 112.014) (width 0.25) (layer F.Cu) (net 6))
 (via (at 116.84 112.014) (size 0.6) (drill 0.4) (layers F.Cu B.Cu) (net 6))
 (segment (start 106.807 108.839) (end 109.093 108.839) (width 0.25) (layer B.Cu) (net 6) (status 10))
 (segment (start 109.093 108.839) (end 112.268 112.014) (width 0.25) (layer B.Cu) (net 6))
 (segment (start 112.268 112.014) (end 116.84 112.014) (width 0.25) (layer B.Cu) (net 6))
 (segment (start 107.315 117.221) (end 107.061 117.475) (width 0.25) (layer B.Cu) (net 6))
 (segment (start 107.188 108.458) (end 106.807 108.839) (width 0.25) (layer B.Cu) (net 6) (status 30))
 (segment (start 116.84 108.372) (end 116.84 101.992) (width 0.25) (layer F.Cu) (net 6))
 (segment (start 143.732 118.332) (end 143.732 119.888) (width 0.25) (layer B.Cu) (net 6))
 (segment (start 142.285999 116.885999) (end 143.732 118.332) (width 0.25) (layer B.Cu) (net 6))
 (segment (start 128.315999 116.885999) (end 142.285999 116.885999) (width 0.25) (layer B.Cu) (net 6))
 (segment (start 128.016 116.586) (end 128.315999 116.885999) (width 0.25) (layer B.Cu) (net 6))
 (segment (start 106.553 92.456) (end 106.553 101.854) (width 0.25) (layer F.Cu) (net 42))
 (segment (start 106.553 101.854) (end 106.807 102.108) (width 0.25) (layer F.Cu) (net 42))
 (segment (start 124.6124 113.4491) (end 126.3142 113.4491) (width 0.25) (layer F.Cu) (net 42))
 (segment (start 115.12 108.372) (end 115.12 112.464) (width 0.25) (layer F.Cu) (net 42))
 (segment (start 116.1051 113.4491) (end 124.6124 113.4491) (width 0.25) (layer F.Cu) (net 42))
 (segment (start 115.12 112.464) (end 116.1051 113.4491) (width 0.25) (layer F.Cu) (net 42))
 (segment (start 113.4 108.372) (end 115.12 108.372) (width 0.25) (layer F.Cu) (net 42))
 (segment (start 113.4 108.372) (end 113.4 117.083) (width 0.25) (layer F.Cu) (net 42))
 (segment (start 113.4 117.083) (end 113.792 117.475) (width 0.25) (layer F.Cu) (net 42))
 (segment (start 106.807 102.108) (end 106.807 102.287) (width 0.25) (layer F.Cu) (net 42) (status 30))
 (segment (start 106.807 102.287) (end 113.4 108.372) (width 0.25) (layer F.Cu) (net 42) (status 10))
 (segment (start 150.406999 119.213001) (end 150.406999 119.087001) (width 0.25) (layer B.Cu) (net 3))
 (segment (start 149.732 119.888) (end 150.406999 119.213001) (width 0.25) (layer B.Cu) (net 3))
 (segment (start 150.406999 119.087001) (end 152.4 117.094) (width 0.25) (layer B.Cu) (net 3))
 (segment (start 158.9056 117.094) (end 164.2872 111.7124) (width 0.25) (layer B.Cu) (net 3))
 (segment (start 152.4 117.094) (end 158.9056 117.094) (width 0.25) (layer B.Cu) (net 3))
 (segment (start 129.7178 113.4491) (end 129.7178 118.7958) (width 0.25) (layer F.Cu) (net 7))
 (segment (start 129.7178 118.7958) (end 130.81 119.888) (width 0.25) (layer F.Cu) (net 7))
 (segment (start 130.9878 119.7102) (end 130.81 119.888) (width 0.25) (layer F.Cu) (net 7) (status 30))
 (segment (start 130.81 119.888) (end 132.81 119.888) (width 0.25) (layer F.Cu) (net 7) (status 30))
 (segment (start 132.81 119.888) (end 142.24 119.888) (width 0.25) (layer F.Cu) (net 7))
 (segment (start 158.8516 118.364) (end 164.2872 112.9284) (width 0.25) (layer B.Cu) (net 2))
 (segment (start 152.301406 118.364) (end 158.8516 118.364) (width 0.25) (layer B.Cu) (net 2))
 (segment (start 151.732 118.933406) (end 152.301406 118.364) (width 0.25) (layer B.Cu) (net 2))
 (segment (start 151.732 119.888) (end 151.732 118.933406) (width 0.25) (layer B.Cu) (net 2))
 (segment (start 158.5436 119.888) (end 164.2872 114.1444) (width 0.25) (layer B.Cu) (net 1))
 (segment (start 153.732 119.888) (end 158.5436 119.888) (width 0.25) (layer B.Cu) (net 1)))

